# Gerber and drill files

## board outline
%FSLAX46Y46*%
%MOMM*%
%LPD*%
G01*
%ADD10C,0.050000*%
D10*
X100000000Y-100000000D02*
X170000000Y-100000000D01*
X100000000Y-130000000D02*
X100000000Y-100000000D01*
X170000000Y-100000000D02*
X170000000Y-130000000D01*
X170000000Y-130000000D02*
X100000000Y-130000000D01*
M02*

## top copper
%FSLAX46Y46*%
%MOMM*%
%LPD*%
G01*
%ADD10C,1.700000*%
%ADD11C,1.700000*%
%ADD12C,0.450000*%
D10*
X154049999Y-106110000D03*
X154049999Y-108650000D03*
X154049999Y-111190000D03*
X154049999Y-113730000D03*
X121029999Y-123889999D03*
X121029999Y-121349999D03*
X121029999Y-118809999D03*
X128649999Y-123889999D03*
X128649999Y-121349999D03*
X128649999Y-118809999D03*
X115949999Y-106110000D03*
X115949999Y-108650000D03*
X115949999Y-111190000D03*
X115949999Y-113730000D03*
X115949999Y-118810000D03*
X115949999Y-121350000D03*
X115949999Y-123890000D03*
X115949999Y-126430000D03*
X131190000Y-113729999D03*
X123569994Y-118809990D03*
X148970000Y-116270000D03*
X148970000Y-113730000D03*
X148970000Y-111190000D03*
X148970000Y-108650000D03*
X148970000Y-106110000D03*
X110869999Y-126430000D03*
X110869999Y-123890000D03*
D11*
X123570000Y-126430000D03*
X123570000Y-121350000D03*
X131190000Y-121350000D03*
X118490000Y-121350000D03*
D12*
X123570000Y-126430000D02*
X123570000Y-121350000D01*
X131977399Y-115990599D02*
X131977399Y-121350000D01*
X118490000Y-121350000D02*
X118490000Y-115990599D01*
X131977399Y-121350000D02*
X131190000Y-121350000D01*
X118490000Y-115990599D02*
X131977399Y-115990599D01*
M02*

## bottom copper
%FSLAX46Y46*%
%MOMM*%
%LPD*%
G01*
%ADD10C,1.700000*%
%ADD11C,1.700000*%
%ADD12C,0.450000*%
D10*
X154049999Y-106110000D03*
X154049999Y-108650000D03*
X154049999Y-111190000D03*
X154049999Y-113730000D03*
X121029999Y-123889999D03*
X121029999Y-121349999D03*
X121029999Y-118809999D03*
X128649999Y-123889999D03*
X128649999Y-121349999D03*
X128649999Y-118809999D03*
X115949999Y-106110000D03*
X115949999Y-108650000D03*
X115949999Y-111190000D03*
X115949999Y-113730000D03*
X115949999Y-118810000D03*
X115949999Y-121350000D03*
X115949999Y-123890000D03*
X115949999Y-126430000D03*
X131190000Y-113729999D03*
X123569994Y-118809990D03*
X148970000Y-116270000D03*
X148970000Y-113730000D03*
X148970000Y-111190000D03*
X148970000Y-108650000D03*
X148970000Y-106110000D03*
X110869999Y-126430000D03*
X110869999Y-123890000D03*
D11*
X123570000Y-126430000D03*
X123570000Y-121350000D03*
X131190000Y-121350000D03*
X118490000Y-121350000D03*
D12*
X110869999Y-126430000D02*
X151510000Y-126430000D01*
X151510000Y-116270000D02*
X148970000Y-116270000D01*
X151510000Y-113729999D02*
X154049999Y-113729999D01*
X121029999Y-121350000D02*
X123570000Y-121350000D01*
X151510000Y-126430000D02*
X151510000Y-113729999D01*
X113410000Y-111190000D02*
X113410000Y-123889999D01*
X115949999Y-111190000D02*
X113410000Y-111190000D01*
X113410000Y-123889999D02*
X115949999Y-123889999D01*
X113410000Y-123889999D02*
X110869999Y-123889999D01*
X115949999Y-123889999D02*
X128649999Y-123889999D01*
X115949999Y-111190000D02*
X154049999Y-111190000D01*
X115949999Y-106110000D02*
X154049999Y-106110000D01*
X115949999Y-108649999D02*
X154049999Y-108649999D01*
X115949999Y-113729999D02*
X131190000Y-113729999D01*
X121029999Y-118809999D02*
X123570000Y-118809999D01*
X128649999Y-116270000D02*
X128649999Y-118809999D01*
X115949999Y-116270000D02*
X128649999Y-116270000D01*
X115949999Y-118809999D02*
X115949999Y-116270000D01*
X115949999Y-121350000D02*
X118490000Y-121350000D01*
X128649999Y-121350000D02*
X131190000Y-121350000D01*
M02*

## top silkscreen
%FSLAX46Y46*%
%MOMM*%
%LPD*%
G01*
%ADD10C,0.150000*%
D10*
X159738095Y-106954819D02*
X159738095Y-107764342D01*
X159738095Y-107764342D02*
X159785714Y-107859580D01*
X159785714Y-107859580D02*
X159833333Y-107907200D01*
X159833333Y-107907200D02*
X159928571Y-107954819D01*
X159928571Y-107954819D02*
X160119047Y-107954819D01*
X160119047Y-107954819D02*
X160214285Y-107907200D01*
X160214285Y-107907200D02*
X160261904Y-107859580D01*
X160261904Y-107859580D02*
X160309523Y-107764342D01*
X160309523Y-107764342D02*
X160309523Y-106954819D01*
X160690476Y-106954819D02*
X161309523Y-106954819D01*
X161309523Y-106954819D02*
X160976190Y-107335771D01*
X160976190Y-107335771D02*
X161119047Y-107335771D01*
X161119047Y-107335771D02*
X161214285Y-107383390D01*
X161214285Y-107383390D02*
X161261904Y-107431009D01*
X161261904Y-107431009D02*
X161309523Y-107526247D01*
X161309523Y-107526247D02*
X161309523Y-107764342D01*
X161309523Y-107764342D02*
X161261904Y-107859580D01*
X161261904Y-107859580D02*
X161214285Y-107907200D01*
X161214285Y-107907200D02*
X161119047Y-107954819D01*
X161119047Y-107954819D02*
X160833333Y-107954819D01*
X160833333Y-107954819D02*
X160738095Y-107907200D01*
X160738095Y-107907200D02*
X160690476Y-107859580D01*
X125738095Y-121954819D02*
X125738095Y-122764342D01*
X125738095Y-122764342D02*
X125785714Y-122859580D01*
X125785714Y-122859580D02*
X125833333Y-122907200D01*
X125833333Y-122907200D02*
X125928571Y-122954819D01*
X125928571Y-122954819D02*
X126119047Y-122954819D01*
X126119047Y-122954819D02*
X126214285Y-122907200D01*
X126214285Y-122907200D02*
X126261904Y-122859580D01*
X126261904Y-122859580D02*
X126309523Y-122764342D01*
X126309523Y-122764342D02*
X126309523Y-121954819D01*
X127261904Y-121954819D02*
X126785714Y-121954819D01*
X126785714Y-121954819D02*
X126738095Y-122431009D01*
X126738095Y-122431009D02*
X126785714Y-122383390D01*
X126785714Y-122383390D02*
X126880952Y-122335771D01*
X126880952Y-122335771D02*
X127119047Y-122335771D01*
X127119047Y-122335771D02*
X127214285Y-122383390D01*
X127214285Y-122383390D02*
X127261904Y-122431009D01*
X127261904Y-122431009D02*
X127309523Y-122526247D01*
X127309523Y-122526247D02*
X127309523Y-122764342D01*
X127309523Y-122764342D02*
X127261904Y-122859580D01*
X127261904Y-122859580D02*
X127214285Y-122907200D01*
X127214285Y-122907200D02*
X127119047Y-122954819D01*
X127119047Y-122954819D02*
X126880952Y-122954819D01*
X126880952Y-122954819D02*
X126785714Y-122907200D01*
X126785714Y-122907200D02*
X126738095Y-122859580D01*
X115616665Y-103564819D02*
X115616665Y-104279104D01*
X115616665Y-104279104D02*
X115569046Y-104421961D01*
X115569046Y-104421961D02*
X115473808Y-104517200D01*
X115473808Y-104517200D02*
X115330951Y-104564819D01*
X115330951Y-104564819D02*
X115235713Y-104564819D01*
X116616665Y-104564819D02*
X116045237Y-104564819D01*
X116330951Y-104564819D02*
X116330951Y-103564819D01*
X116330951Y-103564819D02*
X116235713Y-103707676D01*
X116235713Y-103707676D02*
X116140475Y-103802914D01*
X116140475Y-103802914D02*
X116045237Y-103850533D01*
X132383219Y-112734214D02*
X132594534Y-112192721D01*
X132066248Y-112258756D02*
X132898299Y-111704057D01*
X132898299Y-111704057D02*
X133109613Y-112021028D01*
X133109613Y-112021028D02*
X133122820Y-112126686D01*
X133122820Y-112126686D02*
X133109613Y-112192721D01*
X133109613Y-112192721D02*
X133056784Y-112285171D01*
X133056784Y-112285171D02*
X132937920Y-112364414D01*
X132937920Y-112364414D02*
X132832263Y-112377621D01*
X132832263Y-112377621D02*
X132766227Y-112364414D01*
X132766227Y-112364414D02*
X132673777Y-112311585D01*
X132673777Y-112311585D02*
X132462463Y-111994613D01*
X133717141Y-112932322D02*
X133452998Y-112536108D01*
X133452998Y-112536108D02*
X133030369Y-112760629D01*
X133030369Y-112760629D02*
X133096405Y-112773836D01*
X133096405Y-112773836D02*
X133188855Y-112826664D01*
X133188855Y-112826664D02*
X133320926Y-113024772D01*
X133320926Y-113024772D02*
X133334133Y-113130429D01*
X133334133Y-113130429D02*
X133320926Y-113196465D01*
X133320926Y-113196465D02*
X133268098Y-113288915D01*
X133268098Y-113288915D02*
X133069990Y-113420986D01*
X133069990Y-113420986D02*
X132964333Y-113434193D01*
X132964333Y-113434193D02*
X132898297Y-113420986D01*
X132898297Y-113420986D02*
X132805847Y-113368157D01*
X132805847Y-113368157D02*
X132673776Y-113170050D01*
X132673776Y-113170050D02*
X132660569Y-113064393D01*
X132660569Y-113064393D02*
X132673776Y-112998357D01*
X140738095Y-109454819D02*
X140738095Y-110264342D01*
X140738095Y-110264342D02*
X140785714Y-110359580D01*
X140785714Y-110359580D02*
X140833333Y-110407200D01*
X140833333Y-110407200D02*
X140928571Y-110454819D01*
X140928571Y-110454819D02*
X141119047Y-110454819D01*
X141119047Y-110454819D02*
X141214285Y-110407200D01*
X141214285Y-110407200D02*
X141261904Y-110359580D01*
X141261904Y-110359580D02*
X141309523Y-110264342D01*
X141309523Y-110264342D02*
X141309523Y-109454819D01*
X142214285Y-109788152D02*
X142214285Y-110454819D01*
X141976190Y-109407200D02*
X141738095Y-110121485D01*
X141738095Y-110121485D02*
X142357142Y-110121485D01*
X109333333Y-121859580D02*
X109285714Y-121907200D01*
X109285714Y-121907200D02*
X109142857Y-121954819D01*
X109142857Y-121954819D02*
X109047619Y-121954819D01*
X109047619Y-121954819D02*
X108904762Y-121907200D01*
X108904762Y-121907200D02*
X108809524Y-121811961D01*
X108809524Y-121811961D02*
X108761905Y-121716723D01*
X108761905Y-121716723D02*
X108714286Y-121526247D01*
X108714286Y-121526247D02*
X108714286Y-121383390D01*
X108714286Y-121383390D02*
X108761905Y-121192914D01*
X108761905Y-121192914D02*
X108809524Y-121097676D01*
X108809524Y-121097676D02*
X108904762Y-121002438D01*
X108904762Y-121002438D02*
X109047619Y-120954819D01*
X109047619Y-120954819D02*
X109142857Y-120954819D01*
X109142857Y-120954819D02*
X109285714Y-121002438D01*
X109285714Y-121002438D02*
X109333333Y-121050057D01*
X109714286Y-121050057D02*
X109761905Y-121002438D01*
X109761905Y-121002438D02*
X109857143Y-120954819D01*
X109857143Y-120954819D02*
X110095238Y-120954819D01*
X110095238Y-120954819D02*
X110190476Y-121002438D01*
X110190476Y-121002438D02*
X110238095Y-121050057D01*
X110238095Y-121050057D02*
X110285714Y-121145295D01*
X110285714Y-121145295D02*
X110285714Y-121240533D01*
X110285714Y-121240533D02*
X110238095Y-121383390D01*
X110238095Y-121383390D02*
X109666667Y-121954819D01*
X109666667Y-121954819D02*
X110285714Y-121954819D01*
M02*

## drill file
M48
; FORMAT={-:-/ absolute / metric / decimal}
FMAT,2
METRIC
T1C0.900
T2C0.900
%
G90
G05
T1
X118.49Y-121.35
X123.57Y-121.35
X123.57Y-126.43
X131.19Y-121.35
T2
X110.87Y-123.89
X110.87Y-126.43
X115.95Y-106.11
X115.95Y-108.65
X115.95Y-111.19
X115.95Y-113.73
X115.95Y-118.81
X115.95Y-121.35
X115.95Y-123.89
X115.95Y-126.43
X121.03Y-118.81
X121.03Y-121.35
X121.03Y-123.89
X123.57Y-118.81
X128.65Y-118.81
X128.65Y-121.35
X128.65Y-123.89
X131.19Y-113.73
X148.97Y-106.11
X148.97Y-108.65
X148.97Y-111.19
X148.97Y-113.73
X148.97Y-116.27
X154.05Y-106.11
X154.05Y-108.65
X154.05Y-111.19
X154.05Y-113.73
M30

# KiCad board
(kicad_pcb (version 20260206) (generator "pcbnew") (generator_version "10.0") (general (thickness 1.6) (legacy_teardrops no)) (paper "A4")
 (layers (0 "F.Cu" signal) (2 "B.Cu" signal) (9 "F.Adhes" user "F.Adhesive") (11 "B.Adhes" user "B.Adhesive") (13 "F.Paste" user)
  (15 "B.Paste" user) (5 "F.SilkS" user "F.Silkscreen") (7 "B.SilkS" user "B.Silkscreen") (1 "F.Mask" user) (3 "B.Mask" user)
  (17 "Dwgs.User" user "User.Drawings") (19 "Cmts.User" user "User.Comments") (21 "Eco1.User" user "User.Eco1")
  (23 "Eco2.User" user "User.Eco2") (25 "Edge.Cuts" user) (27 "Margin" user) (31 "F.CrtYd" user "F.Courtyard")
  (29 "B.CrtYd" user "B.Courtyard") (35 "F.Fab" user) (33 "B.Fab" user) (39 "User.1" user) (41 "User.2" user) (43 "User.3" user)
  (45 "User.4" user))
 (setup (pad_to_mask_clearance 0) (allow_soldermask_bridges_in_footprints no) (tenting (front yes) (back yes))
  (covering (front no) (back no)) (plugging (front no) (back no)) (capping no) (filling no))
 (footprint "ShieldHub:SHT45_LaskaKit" (layer "F.Cu") (at 154.049999 106.11)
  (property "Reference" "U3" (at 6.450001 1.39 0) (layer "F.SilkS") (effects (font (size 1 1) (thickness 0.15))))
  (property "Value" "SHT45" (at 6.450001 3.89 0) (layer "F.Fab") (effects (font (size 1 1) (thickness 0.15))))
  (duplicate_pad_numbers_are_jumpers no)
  (pad "1" thru_hole circle (at 0 0) (size 1.7 1.7) (drill 0.9) (layers "*.Cu" "*.Mask") (remove_unused_layers no) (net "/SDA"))
  (pad "2" thru_hole circle (at 0 2.54) (size 1.7 1.7) (drill 0.9) (layers "*.Cu" "*.Mask") (remove_unused_layers no) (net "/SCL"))
  (pad "3" thru_hole circle (at 0 5.08) (size 1.7 1.7) (drill 0.9) (layers "*.Cu" "*.Mask") (remove_unused_layers no) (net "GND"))
  (pad "4" thru_hole circle (at 0 7.62) (size 1.7 1.7) (drill 0.9) (layers "*.Cu" "*.Mask") (remove_unused_layers no) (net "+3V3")))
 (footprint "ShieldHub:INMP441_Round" (layer "F.Cu") (at 128.649999 123.889999)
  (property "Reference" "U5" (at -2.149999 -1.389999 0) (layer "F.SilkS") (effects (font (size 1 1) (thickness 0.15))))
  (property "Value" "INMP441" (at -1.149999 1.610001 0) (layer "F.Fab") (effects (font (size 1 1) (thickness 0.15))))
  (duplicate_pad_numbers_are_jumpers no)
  (pad "1" thru_hole circle (at -7.62 0) (size 1.7 1.7) (drill 0.9) (layers "*.Cu" "*.Mask") (remove_unused_layers no) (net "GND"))
  (pad "2" thru_hole circle (at -7.62 -2.54) (size 1.7 1.7) (drill 0.9) (layers "*.Cu" "*.Mask") (remove_unused_layers no) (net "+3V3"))
  (pad "3" thru_hole circle (at -7.62 -5.08) (size 1.7 1.7) (drill 0.9) (layers "*.Cu" "*.Mask") (remove_unused_layers no) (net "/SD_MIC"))
  (pad "4" thru_hole circle (at 0 0) (size 1.7 1.7) (drill 0.9) (layers "*.Cu" "*.Mask") (remove_unused_layers no) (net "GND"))
  (pad "5" thru_hole circle (at 0 -2.54) (size 1.7 1.7) (drill 0.9) (layers "*.Cu" "*.Mask") (remove_unused_layers no) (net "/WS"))
  (pad "6" thru_hole circle (at 0 -5.08) (size 1.7 1.7) (drill 0.9) (layers "*.Cu" "*.Mask") (remove_unused_layers no) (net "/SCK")))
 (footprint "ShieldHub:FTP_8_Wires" (layer "F.Cu") (at 115.949999 106.11)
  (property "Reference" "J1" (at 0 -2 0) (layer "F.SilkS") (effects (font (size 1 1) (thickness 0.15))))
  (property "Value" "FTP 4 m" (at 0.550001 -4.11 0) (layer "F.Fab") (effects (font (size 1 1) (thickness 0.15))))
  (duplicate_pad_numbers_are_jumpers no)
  (pad "1" thru_hole circle (at 0 0) (size 1.7 1.7) (drill 0.9) (layers "*.Cu" "*.Mask") (remove_unused_layers no) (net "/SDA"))
  (pad "2" thru_hole circle (at 0 2.54) (size 1.7 1.7) (drill 0.9) (layers "*.Cu" "*.Mask") (remove_unused_layers no) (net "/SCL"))
  (pad "3" thru_hole circle (at 0 5.08) (size 1.7 1.7) (drill 0.9) (layers "*.Cu" "*.Mask") (remove_unused_layers no) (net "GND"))
  (pad "4" thru_hole circle (at 0 7.62) (size 1.7 1.7) (drill 0.9) (layers "*.Cu" "*.Mask") (remove_unused_layers no) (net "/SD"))
  (pad "5" thru_hole circle (at 0 12.7) (size 1.7 1.7) (drill 0.9) (layers "*.Cu" "*.Mask") (remove_unused_layers no) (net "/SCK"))
  (pad "6" thru_hole circle (at 0 15.24) (size 1.7 1.7) (drill 0.9) (layers "*.Cu" "*.Mask") (remove_unused_layers no) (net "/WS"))
  (pad "7" thru_hole circle (at 0 17.78) (size 1.7 1.7) (drill 0.9) (layers "*.Cu" "*.Mask") (remove_unused_layers no) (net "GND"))
  (pad "8" thru_hole circle (at 0 20.32) (size 1.7 1.7) (drill 0.9) (layers "*.Cu" "*.Mask") (remove_unused_layers no) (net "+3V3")))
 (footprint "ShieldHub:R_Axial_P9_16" (layer "F.Cu") (at 131.19 113.729999 -56.31)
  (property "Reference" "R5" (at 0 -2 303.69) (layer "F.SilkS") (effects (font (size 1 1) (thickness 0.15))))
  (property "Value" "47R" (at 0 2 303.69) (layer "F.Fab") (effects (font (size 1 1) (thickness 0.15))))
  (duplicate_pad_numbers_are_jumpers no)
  (pad "1" thru_hole circle (at 0 0 303.69) (size 1.7 1.7) (drill 0.9) (layers "*.Cu" "*.Mask") (remove_unused_layers no) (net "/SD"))
  (pad "2" thru_hole circle (at 0 9.1581 303.69) (size 1.7 1.7) (drill 0.9) (layers "*.Cu" "*.Mask") (remove_unused_layers no)
   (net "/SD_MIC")))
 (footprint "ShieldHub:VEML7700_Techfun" (layer "F.Cu") (at 148.97 116.27)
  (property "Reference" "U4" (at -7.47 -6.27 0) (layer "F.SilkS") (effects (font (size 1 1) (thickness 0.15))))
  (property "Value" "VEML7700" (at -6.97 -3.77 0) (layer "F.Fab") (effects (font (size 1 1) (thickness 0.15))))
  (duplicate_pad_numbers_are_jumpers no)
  (pad "1" thru_hole circle (at 0 0) (size 1.7 1.7) (drill 0.9) (layers "*.Cu" "*.Mask") (remove_unused_layers no) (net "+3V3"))
  (pad "2" thru_hole circle (at 0 -2.54) (size 1.7 1.7) (drill 0.9) (layers "*.Cu" "*.Mask") (remove_unused_layers no)
   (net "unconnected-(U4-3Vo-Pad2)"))
  (pad "3" thru_hole circle (at 0 -5.08) (size 1.7 1.7) (drill 0.9) (layers "*.Cu" "*.Mask") (remove_unused_layers no) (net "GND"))
  (pad "4" thru_hole circle (at 0 -7.62) (size 1.7 1.7) (drill 0.9) (layers "*.Cu" "*.Mask") (remove_unused_layers no) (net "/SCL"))
  (pad "5" thru_hole circle (at 0 -10.16) (size 1.7 1.7) (drill 0.9) (layers "*.Cu" "*.Mask") (remove_unused_layers no) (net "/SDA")))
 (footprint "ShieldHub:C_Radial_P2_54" (layer "F.Cu") (at 110.869999 126.43)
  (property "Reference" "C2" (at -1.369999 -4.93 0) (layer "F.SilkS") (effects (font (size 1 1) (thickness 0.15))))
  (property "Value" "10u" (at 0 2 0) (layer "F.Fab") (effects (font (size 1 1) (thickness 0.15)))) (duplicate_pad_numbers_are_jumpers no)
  (pad "1" thru_hole circle (at 0 0) (size 1.7 1.7) (drill 0.9) (layers "*.Cu" "*.Mask") (remove_unused_layers no) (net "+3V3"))
  (pad "2" thru_hole circle (at 0 -2.54) (size 1.7 1.7) (drill 0.9) (layers "*.Cu" "*.Mask") (remove_unused_layers no) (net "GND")))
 (gr_line (start 100 100) (end 170 100) (stroke (width 0.05) (type default)) (layer "Edge.Cuts"))
 (gr_line (start 100 130) (end 100 100) (stroke (width 0.05) (type default)) (layer "Edge.Cuts"))
 (gr_line (start 170 100) (end 170 130) (stroke (width 0.05) (type default)) (layer "Edge.Cuts"))
 (gr_line (start 170 130) (end 100 130) (stroke (width 0.05) (type default)) (layer "Edge.Cuts"))
 (segment (start 123.57 126.43) (end 123.57 121.35) (width 0.45) (layer "F.Cu") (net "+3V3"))
 (via (at 123.57 126.43) (size 1.7) (drill 0.9) (layers "F.Cu" "B.Cu") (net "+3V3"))
 (via (at 123.57 121.35) (size 1.7) (drill 0.9) (layers "F.Cu" "B.Cu") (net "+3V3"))
 (segment (start 110.869999 126.43) (end 151.51 126.43) (width 0.45) (layer "B.Cu") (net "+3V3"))
 (segment (start 151.51 116.27) (end 148.97 116.27) (width 0.45) (layer "B.Cu") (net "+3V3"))
 (segment (start 151.51 113.729999) (end 154.049999 113.729999) (width 0.45) (layer "B.Cu") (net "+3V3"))
 (segment (start 121.029999 121.35) (end 123.57 121.35) (width 0.45) (layer "B.Cu") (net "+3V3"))
 (segment (start 151.51 126.43) (end 151.51 113.729999) (width 0.45) (layer "B.Cu") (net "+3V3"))
 (segment (start 113.41 111.19) (end 113.41 123.889999) (width 0.45) (layer "B.Cu") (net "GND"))
 (segment (start 115.949999 111.19) (end 113.41 111.19) (width 0.45) (layer "B.Cu") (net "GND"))
 (segment (start 113.41 123.889999) (end 115.949999 123.889999) (width 0.45) (layer "B.Cu") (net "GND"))
 (segment (start 113.41 123.889999) (end 110.869999 123.889999) (width 0.45) (layer "B.Cu") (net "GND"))
 (segment (start 115.949999 123.889999) (end 128.649999 123.889999) (width 0.45) (layer "B.Cu") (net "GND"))
 (segment (start 115.949999 111.19) (end 154.049999 111.19) (width 0.45) (layer "B.Cu") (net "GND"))
 (segment (start 115.949999 106.11) (end 154.049999 106.11) (width 0.45) (layer "B.Cu") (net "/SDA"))
 (segment (start 115.949999 108.649999) (end 154.049999 108.649999) (width 0.45) (layer "B.Cu") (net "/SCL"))
 (segment (start 115.949999 113.729999) (end 131.19 113.729999) (width 0.45) (layer "B.Cu") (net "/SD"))
 (segment (start 121.029999 118.809999) (end 123.57 118.809999) (width 0.45) (layer "B.Cu") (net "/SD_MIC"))
 (segment (start 128.649999 116.27) (end 128.649999 118.809999) (width 0.45) (layer "B.Cu") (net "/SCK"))
 (segment (start 115.949999 116.27) (end 128.649999 116.27) (width 0.45) (layer "B.Cu") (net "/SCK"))
 (segment (start 115.949999 118.809999) (end 115.949999 116.27) (width 0.45) (layer "B.Cu") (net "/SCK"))
 (segment (start 131.977399 115.990599) (end 131.977399 121.35) (width 0.45) (layer "F.Cu") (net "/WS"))
 (segment (start 118.49 121.35) (end 118.49 115.990599) (width 0.45) (layer "F.Cu") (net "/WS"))
 (segment (start 131.977399 121.35) (end 131.19 121.35) (width 0.45) (layer "F.Cu") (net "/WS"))
 (segment (start 118.49 115.990599) (end 131.977399 115.990599) (width 0.45) (layer "F.Cu") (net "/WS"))
 (via (at 131.19 121.35) (size 1.7) (drill 0.9) (layers "F.Cu" "B.Cu") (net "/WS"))
 (via (at 118.49 121.35) (size 1.7) (drill 0.9) (layers "F.Cu" "B.Cu") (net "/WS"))
 (segment (start 115.949999 121.35) (end 118.49 121.35) (width 0.45) (layer "B.Cu") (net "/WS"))
 (segment (start 128.649999 121.35) (end 131.19 121.35) (width 0.45) (layer "B.Cu") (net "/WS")))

